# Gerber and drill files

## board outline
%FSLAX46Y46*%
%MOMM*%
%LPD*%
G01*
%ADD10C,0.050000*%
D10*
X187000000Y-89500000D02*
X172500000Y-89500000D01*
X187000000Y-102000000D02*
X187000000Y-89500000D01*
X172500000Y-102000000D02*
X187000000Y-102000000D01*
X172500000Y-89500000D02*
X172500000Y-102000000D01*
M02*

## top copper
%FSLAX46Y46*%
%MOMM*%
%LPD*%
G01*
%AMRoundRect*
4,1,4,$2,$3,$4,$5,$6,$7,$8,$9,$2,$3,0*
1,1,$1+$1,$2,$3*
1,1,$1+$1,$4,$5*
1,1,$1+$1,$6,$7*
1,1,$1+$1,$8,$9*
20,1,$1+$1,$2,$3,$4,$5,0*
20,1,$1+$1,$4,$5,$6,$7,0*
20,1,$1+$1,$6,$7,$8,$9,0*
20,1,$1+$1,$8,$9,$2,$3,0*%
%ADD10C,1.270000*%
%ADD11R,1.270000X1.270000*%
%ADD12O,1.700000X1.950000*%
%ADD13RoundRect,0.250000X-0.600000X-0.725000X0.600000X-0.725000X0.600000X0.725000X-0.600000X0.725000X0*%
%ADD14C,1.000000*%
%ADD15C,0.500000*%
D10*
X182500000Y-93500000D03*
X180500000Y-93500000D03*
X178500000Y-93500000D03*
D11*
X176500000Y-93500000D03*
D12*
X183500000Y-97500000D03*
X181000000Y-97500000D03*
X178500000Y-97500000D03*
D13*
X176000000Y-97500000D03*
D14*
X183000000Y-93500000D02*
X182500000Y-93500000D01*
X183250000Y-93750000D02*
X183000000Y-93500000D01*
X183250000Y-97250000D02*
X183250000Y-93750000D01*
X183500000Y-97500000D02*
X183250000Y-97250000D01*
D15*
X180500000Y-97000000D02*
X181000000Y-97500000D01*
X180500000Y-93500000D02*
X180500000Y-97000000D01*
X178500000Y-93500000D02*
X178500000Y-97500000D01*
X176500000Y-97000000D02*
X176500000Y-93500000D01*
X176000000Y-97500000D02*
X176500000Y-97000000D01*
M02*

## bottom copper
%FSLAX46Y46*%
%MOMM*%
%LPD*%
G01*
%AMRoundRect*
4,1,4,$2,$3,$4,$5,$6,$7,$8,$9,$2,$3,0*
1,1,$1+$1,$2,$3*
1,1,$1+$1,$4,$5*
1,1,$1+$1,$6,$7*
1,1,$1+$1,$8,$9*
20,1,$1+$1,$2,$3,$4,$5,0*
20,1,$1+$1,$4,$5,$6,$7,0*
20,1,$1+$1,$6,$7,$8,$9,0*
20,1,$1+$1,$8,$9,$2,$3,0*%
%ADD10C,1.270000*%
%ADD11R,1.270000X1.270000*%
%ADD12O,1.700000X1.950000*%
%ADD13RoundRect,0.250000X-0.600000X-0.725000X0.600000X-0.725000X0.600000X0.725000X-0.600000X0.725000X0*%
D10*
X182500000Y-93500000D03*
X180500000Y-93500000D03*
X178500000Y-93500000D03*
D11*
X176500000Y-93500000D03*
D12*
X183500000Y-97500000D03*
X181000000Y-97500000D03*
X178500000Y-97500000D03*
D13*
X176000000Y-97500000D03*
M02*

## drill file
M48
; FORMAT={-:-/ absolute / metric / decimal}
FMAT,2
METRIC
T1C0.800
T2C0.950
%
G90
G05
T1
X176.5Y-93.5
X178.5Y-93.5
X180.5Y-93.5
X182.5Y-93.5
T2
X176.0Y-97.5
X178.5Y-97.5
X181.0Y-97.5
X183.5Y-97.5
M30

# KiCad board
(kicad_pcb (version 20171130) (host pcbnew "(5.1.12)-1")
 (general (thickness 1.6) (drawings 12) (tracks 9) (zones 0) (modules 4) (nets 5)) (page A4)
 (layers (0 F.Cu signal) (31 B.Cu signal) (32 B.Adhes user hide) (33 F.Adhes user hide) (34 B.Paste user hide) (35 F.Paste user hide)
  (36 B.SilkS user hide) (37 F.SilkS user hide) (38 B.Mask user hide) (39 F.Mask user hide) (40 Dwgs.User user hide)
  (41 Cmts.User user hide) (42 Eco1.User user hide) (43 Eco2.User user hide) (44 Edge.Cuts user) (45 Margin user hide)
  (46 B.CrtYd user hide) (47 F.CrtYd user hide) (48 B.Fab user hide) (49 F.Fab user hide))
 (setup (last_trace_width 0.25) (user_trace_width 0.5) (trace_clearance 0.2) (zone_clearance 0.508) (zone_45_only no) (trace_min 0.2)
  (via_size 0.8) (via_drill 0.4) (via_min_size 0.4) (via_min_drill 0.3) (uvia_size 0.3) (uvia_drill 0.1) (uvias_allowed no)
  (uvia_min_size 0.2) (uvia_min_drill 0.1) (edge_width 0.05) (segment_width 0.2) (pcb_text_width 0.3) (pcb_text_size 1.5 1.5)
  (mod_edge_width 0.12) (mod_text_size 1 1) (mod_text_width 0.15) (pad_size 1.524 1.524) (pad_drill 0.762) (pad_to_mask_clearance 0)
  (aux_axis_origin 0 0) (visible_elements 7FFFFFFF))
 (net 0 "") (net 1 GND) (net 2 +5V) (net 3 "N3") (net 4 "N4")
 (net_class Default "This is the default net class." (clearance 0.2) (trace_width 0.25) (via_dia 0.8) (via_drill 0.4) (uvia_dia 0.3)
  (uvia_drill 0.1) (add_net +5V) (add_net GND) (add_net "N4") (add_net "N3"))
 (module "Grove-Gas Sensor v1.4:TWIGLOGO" (layer B.Cu) (at 184.5 94)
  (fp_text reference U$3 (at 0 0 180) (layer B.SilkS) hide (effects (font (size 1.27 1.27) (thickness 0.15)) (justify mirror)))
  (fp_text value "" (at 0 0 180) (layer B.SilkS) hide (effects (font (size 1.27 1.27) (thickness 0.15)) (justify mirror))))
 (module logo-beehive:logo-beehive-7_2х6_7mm (layer F.Cu) (at 176 93.5 270)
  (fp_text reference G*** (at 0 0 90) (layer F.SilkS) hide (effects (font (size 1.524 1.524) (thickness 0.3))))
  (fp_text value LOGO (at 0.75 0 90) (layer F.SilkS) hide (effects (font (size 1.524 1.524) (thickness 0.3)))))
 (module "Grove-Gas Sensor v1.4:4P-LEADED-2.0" (layer B.Cu) (at 179.5 93.5)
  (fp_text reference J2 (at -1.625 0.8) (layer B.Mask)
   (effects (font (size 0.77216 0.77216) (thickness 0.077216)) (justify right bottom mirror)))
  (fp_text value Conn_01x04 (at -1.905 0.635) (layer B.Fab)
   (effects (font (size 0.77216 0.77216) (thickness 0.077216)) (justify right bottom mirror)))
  (pad 4 thru_hole circle (at 3 0) (size 1.27 1.27) (drill 0.8) (layers *.Cu *.Mask) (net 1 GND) (solder_mask_margin 0.0508))
  (pad 3 thru_hole circle (at 1 0) (size 1.27 1.27) (drill 0.8) (layers *.Cu *.Mask) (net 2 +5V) (solder_mask_margin 0.0508))
  (pad 2 thru_hole circle (at -1 0) (size 1.27 1.27) (drill 0.8) (layers *.Cu *.Mask) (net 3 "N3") (solder_mask_margin 0.0508))
  (pad 1 thru_hole rect (at -3 0) (size 1.27 1.27) (drill 0.8) (layers *.Cu *.Mask) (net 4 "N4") (solder_mask_margin 0.0508)))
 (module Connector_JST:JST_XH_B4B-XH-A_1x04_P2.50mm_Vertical (layer F.Cu) (at 176 97.5)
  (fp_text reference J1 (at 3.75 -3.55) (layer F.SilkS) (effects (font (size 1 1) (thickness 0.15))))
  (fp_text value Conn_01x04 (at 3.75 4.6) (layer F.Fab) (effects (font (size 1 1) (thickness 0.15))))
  (pad 4 thru_hole oval (at 7.5 0) (size 1.7 1.95) (drill 0.95) (layers *.Cu *.Mask) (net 1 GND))
  (pad 3 thru_hole oval (at 5 0) (size 1.7 1.95) (drill 0.95) (layers *.Cu *.Mask) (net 2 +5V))
  (pad 2 thru_hole oval (at 2.5 0) (size 1.7 1.95) (drill 0.95) (layers *.Cu *.Mask) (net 3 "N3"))
  (pad 1 thru_hole roundrect (at 0 0) (size 1.7 1.95) (drill 0.95) (layers *.Cu *.Mask) (roundrect_rratio 0.1470588235294118) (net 4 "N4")))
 (gr_line (start 187 89.5) (end 172.5 89.5) (layer Edge.Cuts) (width 0.05))
 (gr_line (start 187 102) (end 187 89.5) (layer Edge.Cuts) (width 0.05))
 (gr_line (start 172.5 102) (end 187 102) (layer Edge.Cuts) (width 0.05))
 (gr_line (start 172.5 89.5) (end 172.5 102) (layer Edge.Cuts) (width 0.05))
 (segment (start 183 93.5) (end 182.5 93.5) (width 1) (layer F.Cu) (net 1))
 (segment (start 183.25 93.75) (end 183 93.5) (width 1) (layer F.Cu) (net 1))
 (segment (start 183.25 97.25) (end 183.25 93.75) (width 1) (layer F.Cu) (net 1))
 (segment (start 183.5 97.5) (end 183.25 97.25) (width 1) (layer F.Cu) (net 1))
 (segment (start 180.5 97) (end 181 97.5) (width 0.5) (layer F.Cu) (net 2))
 (segment (start 180.5 93.5) (end 180.5 97) (width 0.5) (layer F.Cu) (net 2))
 (segment (start 178.5 93.5) (end 178.5 97.5) (width 0.5) (layer F.Cu) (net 3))
 (segment (start 176.5 97) (end 176.5 93.5) (width 0.5) (layer F.Cu) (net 4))
 (segment (start 176 97.5) (end 176.5 97) (width 0.5) (layer F.Cu) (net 4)))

